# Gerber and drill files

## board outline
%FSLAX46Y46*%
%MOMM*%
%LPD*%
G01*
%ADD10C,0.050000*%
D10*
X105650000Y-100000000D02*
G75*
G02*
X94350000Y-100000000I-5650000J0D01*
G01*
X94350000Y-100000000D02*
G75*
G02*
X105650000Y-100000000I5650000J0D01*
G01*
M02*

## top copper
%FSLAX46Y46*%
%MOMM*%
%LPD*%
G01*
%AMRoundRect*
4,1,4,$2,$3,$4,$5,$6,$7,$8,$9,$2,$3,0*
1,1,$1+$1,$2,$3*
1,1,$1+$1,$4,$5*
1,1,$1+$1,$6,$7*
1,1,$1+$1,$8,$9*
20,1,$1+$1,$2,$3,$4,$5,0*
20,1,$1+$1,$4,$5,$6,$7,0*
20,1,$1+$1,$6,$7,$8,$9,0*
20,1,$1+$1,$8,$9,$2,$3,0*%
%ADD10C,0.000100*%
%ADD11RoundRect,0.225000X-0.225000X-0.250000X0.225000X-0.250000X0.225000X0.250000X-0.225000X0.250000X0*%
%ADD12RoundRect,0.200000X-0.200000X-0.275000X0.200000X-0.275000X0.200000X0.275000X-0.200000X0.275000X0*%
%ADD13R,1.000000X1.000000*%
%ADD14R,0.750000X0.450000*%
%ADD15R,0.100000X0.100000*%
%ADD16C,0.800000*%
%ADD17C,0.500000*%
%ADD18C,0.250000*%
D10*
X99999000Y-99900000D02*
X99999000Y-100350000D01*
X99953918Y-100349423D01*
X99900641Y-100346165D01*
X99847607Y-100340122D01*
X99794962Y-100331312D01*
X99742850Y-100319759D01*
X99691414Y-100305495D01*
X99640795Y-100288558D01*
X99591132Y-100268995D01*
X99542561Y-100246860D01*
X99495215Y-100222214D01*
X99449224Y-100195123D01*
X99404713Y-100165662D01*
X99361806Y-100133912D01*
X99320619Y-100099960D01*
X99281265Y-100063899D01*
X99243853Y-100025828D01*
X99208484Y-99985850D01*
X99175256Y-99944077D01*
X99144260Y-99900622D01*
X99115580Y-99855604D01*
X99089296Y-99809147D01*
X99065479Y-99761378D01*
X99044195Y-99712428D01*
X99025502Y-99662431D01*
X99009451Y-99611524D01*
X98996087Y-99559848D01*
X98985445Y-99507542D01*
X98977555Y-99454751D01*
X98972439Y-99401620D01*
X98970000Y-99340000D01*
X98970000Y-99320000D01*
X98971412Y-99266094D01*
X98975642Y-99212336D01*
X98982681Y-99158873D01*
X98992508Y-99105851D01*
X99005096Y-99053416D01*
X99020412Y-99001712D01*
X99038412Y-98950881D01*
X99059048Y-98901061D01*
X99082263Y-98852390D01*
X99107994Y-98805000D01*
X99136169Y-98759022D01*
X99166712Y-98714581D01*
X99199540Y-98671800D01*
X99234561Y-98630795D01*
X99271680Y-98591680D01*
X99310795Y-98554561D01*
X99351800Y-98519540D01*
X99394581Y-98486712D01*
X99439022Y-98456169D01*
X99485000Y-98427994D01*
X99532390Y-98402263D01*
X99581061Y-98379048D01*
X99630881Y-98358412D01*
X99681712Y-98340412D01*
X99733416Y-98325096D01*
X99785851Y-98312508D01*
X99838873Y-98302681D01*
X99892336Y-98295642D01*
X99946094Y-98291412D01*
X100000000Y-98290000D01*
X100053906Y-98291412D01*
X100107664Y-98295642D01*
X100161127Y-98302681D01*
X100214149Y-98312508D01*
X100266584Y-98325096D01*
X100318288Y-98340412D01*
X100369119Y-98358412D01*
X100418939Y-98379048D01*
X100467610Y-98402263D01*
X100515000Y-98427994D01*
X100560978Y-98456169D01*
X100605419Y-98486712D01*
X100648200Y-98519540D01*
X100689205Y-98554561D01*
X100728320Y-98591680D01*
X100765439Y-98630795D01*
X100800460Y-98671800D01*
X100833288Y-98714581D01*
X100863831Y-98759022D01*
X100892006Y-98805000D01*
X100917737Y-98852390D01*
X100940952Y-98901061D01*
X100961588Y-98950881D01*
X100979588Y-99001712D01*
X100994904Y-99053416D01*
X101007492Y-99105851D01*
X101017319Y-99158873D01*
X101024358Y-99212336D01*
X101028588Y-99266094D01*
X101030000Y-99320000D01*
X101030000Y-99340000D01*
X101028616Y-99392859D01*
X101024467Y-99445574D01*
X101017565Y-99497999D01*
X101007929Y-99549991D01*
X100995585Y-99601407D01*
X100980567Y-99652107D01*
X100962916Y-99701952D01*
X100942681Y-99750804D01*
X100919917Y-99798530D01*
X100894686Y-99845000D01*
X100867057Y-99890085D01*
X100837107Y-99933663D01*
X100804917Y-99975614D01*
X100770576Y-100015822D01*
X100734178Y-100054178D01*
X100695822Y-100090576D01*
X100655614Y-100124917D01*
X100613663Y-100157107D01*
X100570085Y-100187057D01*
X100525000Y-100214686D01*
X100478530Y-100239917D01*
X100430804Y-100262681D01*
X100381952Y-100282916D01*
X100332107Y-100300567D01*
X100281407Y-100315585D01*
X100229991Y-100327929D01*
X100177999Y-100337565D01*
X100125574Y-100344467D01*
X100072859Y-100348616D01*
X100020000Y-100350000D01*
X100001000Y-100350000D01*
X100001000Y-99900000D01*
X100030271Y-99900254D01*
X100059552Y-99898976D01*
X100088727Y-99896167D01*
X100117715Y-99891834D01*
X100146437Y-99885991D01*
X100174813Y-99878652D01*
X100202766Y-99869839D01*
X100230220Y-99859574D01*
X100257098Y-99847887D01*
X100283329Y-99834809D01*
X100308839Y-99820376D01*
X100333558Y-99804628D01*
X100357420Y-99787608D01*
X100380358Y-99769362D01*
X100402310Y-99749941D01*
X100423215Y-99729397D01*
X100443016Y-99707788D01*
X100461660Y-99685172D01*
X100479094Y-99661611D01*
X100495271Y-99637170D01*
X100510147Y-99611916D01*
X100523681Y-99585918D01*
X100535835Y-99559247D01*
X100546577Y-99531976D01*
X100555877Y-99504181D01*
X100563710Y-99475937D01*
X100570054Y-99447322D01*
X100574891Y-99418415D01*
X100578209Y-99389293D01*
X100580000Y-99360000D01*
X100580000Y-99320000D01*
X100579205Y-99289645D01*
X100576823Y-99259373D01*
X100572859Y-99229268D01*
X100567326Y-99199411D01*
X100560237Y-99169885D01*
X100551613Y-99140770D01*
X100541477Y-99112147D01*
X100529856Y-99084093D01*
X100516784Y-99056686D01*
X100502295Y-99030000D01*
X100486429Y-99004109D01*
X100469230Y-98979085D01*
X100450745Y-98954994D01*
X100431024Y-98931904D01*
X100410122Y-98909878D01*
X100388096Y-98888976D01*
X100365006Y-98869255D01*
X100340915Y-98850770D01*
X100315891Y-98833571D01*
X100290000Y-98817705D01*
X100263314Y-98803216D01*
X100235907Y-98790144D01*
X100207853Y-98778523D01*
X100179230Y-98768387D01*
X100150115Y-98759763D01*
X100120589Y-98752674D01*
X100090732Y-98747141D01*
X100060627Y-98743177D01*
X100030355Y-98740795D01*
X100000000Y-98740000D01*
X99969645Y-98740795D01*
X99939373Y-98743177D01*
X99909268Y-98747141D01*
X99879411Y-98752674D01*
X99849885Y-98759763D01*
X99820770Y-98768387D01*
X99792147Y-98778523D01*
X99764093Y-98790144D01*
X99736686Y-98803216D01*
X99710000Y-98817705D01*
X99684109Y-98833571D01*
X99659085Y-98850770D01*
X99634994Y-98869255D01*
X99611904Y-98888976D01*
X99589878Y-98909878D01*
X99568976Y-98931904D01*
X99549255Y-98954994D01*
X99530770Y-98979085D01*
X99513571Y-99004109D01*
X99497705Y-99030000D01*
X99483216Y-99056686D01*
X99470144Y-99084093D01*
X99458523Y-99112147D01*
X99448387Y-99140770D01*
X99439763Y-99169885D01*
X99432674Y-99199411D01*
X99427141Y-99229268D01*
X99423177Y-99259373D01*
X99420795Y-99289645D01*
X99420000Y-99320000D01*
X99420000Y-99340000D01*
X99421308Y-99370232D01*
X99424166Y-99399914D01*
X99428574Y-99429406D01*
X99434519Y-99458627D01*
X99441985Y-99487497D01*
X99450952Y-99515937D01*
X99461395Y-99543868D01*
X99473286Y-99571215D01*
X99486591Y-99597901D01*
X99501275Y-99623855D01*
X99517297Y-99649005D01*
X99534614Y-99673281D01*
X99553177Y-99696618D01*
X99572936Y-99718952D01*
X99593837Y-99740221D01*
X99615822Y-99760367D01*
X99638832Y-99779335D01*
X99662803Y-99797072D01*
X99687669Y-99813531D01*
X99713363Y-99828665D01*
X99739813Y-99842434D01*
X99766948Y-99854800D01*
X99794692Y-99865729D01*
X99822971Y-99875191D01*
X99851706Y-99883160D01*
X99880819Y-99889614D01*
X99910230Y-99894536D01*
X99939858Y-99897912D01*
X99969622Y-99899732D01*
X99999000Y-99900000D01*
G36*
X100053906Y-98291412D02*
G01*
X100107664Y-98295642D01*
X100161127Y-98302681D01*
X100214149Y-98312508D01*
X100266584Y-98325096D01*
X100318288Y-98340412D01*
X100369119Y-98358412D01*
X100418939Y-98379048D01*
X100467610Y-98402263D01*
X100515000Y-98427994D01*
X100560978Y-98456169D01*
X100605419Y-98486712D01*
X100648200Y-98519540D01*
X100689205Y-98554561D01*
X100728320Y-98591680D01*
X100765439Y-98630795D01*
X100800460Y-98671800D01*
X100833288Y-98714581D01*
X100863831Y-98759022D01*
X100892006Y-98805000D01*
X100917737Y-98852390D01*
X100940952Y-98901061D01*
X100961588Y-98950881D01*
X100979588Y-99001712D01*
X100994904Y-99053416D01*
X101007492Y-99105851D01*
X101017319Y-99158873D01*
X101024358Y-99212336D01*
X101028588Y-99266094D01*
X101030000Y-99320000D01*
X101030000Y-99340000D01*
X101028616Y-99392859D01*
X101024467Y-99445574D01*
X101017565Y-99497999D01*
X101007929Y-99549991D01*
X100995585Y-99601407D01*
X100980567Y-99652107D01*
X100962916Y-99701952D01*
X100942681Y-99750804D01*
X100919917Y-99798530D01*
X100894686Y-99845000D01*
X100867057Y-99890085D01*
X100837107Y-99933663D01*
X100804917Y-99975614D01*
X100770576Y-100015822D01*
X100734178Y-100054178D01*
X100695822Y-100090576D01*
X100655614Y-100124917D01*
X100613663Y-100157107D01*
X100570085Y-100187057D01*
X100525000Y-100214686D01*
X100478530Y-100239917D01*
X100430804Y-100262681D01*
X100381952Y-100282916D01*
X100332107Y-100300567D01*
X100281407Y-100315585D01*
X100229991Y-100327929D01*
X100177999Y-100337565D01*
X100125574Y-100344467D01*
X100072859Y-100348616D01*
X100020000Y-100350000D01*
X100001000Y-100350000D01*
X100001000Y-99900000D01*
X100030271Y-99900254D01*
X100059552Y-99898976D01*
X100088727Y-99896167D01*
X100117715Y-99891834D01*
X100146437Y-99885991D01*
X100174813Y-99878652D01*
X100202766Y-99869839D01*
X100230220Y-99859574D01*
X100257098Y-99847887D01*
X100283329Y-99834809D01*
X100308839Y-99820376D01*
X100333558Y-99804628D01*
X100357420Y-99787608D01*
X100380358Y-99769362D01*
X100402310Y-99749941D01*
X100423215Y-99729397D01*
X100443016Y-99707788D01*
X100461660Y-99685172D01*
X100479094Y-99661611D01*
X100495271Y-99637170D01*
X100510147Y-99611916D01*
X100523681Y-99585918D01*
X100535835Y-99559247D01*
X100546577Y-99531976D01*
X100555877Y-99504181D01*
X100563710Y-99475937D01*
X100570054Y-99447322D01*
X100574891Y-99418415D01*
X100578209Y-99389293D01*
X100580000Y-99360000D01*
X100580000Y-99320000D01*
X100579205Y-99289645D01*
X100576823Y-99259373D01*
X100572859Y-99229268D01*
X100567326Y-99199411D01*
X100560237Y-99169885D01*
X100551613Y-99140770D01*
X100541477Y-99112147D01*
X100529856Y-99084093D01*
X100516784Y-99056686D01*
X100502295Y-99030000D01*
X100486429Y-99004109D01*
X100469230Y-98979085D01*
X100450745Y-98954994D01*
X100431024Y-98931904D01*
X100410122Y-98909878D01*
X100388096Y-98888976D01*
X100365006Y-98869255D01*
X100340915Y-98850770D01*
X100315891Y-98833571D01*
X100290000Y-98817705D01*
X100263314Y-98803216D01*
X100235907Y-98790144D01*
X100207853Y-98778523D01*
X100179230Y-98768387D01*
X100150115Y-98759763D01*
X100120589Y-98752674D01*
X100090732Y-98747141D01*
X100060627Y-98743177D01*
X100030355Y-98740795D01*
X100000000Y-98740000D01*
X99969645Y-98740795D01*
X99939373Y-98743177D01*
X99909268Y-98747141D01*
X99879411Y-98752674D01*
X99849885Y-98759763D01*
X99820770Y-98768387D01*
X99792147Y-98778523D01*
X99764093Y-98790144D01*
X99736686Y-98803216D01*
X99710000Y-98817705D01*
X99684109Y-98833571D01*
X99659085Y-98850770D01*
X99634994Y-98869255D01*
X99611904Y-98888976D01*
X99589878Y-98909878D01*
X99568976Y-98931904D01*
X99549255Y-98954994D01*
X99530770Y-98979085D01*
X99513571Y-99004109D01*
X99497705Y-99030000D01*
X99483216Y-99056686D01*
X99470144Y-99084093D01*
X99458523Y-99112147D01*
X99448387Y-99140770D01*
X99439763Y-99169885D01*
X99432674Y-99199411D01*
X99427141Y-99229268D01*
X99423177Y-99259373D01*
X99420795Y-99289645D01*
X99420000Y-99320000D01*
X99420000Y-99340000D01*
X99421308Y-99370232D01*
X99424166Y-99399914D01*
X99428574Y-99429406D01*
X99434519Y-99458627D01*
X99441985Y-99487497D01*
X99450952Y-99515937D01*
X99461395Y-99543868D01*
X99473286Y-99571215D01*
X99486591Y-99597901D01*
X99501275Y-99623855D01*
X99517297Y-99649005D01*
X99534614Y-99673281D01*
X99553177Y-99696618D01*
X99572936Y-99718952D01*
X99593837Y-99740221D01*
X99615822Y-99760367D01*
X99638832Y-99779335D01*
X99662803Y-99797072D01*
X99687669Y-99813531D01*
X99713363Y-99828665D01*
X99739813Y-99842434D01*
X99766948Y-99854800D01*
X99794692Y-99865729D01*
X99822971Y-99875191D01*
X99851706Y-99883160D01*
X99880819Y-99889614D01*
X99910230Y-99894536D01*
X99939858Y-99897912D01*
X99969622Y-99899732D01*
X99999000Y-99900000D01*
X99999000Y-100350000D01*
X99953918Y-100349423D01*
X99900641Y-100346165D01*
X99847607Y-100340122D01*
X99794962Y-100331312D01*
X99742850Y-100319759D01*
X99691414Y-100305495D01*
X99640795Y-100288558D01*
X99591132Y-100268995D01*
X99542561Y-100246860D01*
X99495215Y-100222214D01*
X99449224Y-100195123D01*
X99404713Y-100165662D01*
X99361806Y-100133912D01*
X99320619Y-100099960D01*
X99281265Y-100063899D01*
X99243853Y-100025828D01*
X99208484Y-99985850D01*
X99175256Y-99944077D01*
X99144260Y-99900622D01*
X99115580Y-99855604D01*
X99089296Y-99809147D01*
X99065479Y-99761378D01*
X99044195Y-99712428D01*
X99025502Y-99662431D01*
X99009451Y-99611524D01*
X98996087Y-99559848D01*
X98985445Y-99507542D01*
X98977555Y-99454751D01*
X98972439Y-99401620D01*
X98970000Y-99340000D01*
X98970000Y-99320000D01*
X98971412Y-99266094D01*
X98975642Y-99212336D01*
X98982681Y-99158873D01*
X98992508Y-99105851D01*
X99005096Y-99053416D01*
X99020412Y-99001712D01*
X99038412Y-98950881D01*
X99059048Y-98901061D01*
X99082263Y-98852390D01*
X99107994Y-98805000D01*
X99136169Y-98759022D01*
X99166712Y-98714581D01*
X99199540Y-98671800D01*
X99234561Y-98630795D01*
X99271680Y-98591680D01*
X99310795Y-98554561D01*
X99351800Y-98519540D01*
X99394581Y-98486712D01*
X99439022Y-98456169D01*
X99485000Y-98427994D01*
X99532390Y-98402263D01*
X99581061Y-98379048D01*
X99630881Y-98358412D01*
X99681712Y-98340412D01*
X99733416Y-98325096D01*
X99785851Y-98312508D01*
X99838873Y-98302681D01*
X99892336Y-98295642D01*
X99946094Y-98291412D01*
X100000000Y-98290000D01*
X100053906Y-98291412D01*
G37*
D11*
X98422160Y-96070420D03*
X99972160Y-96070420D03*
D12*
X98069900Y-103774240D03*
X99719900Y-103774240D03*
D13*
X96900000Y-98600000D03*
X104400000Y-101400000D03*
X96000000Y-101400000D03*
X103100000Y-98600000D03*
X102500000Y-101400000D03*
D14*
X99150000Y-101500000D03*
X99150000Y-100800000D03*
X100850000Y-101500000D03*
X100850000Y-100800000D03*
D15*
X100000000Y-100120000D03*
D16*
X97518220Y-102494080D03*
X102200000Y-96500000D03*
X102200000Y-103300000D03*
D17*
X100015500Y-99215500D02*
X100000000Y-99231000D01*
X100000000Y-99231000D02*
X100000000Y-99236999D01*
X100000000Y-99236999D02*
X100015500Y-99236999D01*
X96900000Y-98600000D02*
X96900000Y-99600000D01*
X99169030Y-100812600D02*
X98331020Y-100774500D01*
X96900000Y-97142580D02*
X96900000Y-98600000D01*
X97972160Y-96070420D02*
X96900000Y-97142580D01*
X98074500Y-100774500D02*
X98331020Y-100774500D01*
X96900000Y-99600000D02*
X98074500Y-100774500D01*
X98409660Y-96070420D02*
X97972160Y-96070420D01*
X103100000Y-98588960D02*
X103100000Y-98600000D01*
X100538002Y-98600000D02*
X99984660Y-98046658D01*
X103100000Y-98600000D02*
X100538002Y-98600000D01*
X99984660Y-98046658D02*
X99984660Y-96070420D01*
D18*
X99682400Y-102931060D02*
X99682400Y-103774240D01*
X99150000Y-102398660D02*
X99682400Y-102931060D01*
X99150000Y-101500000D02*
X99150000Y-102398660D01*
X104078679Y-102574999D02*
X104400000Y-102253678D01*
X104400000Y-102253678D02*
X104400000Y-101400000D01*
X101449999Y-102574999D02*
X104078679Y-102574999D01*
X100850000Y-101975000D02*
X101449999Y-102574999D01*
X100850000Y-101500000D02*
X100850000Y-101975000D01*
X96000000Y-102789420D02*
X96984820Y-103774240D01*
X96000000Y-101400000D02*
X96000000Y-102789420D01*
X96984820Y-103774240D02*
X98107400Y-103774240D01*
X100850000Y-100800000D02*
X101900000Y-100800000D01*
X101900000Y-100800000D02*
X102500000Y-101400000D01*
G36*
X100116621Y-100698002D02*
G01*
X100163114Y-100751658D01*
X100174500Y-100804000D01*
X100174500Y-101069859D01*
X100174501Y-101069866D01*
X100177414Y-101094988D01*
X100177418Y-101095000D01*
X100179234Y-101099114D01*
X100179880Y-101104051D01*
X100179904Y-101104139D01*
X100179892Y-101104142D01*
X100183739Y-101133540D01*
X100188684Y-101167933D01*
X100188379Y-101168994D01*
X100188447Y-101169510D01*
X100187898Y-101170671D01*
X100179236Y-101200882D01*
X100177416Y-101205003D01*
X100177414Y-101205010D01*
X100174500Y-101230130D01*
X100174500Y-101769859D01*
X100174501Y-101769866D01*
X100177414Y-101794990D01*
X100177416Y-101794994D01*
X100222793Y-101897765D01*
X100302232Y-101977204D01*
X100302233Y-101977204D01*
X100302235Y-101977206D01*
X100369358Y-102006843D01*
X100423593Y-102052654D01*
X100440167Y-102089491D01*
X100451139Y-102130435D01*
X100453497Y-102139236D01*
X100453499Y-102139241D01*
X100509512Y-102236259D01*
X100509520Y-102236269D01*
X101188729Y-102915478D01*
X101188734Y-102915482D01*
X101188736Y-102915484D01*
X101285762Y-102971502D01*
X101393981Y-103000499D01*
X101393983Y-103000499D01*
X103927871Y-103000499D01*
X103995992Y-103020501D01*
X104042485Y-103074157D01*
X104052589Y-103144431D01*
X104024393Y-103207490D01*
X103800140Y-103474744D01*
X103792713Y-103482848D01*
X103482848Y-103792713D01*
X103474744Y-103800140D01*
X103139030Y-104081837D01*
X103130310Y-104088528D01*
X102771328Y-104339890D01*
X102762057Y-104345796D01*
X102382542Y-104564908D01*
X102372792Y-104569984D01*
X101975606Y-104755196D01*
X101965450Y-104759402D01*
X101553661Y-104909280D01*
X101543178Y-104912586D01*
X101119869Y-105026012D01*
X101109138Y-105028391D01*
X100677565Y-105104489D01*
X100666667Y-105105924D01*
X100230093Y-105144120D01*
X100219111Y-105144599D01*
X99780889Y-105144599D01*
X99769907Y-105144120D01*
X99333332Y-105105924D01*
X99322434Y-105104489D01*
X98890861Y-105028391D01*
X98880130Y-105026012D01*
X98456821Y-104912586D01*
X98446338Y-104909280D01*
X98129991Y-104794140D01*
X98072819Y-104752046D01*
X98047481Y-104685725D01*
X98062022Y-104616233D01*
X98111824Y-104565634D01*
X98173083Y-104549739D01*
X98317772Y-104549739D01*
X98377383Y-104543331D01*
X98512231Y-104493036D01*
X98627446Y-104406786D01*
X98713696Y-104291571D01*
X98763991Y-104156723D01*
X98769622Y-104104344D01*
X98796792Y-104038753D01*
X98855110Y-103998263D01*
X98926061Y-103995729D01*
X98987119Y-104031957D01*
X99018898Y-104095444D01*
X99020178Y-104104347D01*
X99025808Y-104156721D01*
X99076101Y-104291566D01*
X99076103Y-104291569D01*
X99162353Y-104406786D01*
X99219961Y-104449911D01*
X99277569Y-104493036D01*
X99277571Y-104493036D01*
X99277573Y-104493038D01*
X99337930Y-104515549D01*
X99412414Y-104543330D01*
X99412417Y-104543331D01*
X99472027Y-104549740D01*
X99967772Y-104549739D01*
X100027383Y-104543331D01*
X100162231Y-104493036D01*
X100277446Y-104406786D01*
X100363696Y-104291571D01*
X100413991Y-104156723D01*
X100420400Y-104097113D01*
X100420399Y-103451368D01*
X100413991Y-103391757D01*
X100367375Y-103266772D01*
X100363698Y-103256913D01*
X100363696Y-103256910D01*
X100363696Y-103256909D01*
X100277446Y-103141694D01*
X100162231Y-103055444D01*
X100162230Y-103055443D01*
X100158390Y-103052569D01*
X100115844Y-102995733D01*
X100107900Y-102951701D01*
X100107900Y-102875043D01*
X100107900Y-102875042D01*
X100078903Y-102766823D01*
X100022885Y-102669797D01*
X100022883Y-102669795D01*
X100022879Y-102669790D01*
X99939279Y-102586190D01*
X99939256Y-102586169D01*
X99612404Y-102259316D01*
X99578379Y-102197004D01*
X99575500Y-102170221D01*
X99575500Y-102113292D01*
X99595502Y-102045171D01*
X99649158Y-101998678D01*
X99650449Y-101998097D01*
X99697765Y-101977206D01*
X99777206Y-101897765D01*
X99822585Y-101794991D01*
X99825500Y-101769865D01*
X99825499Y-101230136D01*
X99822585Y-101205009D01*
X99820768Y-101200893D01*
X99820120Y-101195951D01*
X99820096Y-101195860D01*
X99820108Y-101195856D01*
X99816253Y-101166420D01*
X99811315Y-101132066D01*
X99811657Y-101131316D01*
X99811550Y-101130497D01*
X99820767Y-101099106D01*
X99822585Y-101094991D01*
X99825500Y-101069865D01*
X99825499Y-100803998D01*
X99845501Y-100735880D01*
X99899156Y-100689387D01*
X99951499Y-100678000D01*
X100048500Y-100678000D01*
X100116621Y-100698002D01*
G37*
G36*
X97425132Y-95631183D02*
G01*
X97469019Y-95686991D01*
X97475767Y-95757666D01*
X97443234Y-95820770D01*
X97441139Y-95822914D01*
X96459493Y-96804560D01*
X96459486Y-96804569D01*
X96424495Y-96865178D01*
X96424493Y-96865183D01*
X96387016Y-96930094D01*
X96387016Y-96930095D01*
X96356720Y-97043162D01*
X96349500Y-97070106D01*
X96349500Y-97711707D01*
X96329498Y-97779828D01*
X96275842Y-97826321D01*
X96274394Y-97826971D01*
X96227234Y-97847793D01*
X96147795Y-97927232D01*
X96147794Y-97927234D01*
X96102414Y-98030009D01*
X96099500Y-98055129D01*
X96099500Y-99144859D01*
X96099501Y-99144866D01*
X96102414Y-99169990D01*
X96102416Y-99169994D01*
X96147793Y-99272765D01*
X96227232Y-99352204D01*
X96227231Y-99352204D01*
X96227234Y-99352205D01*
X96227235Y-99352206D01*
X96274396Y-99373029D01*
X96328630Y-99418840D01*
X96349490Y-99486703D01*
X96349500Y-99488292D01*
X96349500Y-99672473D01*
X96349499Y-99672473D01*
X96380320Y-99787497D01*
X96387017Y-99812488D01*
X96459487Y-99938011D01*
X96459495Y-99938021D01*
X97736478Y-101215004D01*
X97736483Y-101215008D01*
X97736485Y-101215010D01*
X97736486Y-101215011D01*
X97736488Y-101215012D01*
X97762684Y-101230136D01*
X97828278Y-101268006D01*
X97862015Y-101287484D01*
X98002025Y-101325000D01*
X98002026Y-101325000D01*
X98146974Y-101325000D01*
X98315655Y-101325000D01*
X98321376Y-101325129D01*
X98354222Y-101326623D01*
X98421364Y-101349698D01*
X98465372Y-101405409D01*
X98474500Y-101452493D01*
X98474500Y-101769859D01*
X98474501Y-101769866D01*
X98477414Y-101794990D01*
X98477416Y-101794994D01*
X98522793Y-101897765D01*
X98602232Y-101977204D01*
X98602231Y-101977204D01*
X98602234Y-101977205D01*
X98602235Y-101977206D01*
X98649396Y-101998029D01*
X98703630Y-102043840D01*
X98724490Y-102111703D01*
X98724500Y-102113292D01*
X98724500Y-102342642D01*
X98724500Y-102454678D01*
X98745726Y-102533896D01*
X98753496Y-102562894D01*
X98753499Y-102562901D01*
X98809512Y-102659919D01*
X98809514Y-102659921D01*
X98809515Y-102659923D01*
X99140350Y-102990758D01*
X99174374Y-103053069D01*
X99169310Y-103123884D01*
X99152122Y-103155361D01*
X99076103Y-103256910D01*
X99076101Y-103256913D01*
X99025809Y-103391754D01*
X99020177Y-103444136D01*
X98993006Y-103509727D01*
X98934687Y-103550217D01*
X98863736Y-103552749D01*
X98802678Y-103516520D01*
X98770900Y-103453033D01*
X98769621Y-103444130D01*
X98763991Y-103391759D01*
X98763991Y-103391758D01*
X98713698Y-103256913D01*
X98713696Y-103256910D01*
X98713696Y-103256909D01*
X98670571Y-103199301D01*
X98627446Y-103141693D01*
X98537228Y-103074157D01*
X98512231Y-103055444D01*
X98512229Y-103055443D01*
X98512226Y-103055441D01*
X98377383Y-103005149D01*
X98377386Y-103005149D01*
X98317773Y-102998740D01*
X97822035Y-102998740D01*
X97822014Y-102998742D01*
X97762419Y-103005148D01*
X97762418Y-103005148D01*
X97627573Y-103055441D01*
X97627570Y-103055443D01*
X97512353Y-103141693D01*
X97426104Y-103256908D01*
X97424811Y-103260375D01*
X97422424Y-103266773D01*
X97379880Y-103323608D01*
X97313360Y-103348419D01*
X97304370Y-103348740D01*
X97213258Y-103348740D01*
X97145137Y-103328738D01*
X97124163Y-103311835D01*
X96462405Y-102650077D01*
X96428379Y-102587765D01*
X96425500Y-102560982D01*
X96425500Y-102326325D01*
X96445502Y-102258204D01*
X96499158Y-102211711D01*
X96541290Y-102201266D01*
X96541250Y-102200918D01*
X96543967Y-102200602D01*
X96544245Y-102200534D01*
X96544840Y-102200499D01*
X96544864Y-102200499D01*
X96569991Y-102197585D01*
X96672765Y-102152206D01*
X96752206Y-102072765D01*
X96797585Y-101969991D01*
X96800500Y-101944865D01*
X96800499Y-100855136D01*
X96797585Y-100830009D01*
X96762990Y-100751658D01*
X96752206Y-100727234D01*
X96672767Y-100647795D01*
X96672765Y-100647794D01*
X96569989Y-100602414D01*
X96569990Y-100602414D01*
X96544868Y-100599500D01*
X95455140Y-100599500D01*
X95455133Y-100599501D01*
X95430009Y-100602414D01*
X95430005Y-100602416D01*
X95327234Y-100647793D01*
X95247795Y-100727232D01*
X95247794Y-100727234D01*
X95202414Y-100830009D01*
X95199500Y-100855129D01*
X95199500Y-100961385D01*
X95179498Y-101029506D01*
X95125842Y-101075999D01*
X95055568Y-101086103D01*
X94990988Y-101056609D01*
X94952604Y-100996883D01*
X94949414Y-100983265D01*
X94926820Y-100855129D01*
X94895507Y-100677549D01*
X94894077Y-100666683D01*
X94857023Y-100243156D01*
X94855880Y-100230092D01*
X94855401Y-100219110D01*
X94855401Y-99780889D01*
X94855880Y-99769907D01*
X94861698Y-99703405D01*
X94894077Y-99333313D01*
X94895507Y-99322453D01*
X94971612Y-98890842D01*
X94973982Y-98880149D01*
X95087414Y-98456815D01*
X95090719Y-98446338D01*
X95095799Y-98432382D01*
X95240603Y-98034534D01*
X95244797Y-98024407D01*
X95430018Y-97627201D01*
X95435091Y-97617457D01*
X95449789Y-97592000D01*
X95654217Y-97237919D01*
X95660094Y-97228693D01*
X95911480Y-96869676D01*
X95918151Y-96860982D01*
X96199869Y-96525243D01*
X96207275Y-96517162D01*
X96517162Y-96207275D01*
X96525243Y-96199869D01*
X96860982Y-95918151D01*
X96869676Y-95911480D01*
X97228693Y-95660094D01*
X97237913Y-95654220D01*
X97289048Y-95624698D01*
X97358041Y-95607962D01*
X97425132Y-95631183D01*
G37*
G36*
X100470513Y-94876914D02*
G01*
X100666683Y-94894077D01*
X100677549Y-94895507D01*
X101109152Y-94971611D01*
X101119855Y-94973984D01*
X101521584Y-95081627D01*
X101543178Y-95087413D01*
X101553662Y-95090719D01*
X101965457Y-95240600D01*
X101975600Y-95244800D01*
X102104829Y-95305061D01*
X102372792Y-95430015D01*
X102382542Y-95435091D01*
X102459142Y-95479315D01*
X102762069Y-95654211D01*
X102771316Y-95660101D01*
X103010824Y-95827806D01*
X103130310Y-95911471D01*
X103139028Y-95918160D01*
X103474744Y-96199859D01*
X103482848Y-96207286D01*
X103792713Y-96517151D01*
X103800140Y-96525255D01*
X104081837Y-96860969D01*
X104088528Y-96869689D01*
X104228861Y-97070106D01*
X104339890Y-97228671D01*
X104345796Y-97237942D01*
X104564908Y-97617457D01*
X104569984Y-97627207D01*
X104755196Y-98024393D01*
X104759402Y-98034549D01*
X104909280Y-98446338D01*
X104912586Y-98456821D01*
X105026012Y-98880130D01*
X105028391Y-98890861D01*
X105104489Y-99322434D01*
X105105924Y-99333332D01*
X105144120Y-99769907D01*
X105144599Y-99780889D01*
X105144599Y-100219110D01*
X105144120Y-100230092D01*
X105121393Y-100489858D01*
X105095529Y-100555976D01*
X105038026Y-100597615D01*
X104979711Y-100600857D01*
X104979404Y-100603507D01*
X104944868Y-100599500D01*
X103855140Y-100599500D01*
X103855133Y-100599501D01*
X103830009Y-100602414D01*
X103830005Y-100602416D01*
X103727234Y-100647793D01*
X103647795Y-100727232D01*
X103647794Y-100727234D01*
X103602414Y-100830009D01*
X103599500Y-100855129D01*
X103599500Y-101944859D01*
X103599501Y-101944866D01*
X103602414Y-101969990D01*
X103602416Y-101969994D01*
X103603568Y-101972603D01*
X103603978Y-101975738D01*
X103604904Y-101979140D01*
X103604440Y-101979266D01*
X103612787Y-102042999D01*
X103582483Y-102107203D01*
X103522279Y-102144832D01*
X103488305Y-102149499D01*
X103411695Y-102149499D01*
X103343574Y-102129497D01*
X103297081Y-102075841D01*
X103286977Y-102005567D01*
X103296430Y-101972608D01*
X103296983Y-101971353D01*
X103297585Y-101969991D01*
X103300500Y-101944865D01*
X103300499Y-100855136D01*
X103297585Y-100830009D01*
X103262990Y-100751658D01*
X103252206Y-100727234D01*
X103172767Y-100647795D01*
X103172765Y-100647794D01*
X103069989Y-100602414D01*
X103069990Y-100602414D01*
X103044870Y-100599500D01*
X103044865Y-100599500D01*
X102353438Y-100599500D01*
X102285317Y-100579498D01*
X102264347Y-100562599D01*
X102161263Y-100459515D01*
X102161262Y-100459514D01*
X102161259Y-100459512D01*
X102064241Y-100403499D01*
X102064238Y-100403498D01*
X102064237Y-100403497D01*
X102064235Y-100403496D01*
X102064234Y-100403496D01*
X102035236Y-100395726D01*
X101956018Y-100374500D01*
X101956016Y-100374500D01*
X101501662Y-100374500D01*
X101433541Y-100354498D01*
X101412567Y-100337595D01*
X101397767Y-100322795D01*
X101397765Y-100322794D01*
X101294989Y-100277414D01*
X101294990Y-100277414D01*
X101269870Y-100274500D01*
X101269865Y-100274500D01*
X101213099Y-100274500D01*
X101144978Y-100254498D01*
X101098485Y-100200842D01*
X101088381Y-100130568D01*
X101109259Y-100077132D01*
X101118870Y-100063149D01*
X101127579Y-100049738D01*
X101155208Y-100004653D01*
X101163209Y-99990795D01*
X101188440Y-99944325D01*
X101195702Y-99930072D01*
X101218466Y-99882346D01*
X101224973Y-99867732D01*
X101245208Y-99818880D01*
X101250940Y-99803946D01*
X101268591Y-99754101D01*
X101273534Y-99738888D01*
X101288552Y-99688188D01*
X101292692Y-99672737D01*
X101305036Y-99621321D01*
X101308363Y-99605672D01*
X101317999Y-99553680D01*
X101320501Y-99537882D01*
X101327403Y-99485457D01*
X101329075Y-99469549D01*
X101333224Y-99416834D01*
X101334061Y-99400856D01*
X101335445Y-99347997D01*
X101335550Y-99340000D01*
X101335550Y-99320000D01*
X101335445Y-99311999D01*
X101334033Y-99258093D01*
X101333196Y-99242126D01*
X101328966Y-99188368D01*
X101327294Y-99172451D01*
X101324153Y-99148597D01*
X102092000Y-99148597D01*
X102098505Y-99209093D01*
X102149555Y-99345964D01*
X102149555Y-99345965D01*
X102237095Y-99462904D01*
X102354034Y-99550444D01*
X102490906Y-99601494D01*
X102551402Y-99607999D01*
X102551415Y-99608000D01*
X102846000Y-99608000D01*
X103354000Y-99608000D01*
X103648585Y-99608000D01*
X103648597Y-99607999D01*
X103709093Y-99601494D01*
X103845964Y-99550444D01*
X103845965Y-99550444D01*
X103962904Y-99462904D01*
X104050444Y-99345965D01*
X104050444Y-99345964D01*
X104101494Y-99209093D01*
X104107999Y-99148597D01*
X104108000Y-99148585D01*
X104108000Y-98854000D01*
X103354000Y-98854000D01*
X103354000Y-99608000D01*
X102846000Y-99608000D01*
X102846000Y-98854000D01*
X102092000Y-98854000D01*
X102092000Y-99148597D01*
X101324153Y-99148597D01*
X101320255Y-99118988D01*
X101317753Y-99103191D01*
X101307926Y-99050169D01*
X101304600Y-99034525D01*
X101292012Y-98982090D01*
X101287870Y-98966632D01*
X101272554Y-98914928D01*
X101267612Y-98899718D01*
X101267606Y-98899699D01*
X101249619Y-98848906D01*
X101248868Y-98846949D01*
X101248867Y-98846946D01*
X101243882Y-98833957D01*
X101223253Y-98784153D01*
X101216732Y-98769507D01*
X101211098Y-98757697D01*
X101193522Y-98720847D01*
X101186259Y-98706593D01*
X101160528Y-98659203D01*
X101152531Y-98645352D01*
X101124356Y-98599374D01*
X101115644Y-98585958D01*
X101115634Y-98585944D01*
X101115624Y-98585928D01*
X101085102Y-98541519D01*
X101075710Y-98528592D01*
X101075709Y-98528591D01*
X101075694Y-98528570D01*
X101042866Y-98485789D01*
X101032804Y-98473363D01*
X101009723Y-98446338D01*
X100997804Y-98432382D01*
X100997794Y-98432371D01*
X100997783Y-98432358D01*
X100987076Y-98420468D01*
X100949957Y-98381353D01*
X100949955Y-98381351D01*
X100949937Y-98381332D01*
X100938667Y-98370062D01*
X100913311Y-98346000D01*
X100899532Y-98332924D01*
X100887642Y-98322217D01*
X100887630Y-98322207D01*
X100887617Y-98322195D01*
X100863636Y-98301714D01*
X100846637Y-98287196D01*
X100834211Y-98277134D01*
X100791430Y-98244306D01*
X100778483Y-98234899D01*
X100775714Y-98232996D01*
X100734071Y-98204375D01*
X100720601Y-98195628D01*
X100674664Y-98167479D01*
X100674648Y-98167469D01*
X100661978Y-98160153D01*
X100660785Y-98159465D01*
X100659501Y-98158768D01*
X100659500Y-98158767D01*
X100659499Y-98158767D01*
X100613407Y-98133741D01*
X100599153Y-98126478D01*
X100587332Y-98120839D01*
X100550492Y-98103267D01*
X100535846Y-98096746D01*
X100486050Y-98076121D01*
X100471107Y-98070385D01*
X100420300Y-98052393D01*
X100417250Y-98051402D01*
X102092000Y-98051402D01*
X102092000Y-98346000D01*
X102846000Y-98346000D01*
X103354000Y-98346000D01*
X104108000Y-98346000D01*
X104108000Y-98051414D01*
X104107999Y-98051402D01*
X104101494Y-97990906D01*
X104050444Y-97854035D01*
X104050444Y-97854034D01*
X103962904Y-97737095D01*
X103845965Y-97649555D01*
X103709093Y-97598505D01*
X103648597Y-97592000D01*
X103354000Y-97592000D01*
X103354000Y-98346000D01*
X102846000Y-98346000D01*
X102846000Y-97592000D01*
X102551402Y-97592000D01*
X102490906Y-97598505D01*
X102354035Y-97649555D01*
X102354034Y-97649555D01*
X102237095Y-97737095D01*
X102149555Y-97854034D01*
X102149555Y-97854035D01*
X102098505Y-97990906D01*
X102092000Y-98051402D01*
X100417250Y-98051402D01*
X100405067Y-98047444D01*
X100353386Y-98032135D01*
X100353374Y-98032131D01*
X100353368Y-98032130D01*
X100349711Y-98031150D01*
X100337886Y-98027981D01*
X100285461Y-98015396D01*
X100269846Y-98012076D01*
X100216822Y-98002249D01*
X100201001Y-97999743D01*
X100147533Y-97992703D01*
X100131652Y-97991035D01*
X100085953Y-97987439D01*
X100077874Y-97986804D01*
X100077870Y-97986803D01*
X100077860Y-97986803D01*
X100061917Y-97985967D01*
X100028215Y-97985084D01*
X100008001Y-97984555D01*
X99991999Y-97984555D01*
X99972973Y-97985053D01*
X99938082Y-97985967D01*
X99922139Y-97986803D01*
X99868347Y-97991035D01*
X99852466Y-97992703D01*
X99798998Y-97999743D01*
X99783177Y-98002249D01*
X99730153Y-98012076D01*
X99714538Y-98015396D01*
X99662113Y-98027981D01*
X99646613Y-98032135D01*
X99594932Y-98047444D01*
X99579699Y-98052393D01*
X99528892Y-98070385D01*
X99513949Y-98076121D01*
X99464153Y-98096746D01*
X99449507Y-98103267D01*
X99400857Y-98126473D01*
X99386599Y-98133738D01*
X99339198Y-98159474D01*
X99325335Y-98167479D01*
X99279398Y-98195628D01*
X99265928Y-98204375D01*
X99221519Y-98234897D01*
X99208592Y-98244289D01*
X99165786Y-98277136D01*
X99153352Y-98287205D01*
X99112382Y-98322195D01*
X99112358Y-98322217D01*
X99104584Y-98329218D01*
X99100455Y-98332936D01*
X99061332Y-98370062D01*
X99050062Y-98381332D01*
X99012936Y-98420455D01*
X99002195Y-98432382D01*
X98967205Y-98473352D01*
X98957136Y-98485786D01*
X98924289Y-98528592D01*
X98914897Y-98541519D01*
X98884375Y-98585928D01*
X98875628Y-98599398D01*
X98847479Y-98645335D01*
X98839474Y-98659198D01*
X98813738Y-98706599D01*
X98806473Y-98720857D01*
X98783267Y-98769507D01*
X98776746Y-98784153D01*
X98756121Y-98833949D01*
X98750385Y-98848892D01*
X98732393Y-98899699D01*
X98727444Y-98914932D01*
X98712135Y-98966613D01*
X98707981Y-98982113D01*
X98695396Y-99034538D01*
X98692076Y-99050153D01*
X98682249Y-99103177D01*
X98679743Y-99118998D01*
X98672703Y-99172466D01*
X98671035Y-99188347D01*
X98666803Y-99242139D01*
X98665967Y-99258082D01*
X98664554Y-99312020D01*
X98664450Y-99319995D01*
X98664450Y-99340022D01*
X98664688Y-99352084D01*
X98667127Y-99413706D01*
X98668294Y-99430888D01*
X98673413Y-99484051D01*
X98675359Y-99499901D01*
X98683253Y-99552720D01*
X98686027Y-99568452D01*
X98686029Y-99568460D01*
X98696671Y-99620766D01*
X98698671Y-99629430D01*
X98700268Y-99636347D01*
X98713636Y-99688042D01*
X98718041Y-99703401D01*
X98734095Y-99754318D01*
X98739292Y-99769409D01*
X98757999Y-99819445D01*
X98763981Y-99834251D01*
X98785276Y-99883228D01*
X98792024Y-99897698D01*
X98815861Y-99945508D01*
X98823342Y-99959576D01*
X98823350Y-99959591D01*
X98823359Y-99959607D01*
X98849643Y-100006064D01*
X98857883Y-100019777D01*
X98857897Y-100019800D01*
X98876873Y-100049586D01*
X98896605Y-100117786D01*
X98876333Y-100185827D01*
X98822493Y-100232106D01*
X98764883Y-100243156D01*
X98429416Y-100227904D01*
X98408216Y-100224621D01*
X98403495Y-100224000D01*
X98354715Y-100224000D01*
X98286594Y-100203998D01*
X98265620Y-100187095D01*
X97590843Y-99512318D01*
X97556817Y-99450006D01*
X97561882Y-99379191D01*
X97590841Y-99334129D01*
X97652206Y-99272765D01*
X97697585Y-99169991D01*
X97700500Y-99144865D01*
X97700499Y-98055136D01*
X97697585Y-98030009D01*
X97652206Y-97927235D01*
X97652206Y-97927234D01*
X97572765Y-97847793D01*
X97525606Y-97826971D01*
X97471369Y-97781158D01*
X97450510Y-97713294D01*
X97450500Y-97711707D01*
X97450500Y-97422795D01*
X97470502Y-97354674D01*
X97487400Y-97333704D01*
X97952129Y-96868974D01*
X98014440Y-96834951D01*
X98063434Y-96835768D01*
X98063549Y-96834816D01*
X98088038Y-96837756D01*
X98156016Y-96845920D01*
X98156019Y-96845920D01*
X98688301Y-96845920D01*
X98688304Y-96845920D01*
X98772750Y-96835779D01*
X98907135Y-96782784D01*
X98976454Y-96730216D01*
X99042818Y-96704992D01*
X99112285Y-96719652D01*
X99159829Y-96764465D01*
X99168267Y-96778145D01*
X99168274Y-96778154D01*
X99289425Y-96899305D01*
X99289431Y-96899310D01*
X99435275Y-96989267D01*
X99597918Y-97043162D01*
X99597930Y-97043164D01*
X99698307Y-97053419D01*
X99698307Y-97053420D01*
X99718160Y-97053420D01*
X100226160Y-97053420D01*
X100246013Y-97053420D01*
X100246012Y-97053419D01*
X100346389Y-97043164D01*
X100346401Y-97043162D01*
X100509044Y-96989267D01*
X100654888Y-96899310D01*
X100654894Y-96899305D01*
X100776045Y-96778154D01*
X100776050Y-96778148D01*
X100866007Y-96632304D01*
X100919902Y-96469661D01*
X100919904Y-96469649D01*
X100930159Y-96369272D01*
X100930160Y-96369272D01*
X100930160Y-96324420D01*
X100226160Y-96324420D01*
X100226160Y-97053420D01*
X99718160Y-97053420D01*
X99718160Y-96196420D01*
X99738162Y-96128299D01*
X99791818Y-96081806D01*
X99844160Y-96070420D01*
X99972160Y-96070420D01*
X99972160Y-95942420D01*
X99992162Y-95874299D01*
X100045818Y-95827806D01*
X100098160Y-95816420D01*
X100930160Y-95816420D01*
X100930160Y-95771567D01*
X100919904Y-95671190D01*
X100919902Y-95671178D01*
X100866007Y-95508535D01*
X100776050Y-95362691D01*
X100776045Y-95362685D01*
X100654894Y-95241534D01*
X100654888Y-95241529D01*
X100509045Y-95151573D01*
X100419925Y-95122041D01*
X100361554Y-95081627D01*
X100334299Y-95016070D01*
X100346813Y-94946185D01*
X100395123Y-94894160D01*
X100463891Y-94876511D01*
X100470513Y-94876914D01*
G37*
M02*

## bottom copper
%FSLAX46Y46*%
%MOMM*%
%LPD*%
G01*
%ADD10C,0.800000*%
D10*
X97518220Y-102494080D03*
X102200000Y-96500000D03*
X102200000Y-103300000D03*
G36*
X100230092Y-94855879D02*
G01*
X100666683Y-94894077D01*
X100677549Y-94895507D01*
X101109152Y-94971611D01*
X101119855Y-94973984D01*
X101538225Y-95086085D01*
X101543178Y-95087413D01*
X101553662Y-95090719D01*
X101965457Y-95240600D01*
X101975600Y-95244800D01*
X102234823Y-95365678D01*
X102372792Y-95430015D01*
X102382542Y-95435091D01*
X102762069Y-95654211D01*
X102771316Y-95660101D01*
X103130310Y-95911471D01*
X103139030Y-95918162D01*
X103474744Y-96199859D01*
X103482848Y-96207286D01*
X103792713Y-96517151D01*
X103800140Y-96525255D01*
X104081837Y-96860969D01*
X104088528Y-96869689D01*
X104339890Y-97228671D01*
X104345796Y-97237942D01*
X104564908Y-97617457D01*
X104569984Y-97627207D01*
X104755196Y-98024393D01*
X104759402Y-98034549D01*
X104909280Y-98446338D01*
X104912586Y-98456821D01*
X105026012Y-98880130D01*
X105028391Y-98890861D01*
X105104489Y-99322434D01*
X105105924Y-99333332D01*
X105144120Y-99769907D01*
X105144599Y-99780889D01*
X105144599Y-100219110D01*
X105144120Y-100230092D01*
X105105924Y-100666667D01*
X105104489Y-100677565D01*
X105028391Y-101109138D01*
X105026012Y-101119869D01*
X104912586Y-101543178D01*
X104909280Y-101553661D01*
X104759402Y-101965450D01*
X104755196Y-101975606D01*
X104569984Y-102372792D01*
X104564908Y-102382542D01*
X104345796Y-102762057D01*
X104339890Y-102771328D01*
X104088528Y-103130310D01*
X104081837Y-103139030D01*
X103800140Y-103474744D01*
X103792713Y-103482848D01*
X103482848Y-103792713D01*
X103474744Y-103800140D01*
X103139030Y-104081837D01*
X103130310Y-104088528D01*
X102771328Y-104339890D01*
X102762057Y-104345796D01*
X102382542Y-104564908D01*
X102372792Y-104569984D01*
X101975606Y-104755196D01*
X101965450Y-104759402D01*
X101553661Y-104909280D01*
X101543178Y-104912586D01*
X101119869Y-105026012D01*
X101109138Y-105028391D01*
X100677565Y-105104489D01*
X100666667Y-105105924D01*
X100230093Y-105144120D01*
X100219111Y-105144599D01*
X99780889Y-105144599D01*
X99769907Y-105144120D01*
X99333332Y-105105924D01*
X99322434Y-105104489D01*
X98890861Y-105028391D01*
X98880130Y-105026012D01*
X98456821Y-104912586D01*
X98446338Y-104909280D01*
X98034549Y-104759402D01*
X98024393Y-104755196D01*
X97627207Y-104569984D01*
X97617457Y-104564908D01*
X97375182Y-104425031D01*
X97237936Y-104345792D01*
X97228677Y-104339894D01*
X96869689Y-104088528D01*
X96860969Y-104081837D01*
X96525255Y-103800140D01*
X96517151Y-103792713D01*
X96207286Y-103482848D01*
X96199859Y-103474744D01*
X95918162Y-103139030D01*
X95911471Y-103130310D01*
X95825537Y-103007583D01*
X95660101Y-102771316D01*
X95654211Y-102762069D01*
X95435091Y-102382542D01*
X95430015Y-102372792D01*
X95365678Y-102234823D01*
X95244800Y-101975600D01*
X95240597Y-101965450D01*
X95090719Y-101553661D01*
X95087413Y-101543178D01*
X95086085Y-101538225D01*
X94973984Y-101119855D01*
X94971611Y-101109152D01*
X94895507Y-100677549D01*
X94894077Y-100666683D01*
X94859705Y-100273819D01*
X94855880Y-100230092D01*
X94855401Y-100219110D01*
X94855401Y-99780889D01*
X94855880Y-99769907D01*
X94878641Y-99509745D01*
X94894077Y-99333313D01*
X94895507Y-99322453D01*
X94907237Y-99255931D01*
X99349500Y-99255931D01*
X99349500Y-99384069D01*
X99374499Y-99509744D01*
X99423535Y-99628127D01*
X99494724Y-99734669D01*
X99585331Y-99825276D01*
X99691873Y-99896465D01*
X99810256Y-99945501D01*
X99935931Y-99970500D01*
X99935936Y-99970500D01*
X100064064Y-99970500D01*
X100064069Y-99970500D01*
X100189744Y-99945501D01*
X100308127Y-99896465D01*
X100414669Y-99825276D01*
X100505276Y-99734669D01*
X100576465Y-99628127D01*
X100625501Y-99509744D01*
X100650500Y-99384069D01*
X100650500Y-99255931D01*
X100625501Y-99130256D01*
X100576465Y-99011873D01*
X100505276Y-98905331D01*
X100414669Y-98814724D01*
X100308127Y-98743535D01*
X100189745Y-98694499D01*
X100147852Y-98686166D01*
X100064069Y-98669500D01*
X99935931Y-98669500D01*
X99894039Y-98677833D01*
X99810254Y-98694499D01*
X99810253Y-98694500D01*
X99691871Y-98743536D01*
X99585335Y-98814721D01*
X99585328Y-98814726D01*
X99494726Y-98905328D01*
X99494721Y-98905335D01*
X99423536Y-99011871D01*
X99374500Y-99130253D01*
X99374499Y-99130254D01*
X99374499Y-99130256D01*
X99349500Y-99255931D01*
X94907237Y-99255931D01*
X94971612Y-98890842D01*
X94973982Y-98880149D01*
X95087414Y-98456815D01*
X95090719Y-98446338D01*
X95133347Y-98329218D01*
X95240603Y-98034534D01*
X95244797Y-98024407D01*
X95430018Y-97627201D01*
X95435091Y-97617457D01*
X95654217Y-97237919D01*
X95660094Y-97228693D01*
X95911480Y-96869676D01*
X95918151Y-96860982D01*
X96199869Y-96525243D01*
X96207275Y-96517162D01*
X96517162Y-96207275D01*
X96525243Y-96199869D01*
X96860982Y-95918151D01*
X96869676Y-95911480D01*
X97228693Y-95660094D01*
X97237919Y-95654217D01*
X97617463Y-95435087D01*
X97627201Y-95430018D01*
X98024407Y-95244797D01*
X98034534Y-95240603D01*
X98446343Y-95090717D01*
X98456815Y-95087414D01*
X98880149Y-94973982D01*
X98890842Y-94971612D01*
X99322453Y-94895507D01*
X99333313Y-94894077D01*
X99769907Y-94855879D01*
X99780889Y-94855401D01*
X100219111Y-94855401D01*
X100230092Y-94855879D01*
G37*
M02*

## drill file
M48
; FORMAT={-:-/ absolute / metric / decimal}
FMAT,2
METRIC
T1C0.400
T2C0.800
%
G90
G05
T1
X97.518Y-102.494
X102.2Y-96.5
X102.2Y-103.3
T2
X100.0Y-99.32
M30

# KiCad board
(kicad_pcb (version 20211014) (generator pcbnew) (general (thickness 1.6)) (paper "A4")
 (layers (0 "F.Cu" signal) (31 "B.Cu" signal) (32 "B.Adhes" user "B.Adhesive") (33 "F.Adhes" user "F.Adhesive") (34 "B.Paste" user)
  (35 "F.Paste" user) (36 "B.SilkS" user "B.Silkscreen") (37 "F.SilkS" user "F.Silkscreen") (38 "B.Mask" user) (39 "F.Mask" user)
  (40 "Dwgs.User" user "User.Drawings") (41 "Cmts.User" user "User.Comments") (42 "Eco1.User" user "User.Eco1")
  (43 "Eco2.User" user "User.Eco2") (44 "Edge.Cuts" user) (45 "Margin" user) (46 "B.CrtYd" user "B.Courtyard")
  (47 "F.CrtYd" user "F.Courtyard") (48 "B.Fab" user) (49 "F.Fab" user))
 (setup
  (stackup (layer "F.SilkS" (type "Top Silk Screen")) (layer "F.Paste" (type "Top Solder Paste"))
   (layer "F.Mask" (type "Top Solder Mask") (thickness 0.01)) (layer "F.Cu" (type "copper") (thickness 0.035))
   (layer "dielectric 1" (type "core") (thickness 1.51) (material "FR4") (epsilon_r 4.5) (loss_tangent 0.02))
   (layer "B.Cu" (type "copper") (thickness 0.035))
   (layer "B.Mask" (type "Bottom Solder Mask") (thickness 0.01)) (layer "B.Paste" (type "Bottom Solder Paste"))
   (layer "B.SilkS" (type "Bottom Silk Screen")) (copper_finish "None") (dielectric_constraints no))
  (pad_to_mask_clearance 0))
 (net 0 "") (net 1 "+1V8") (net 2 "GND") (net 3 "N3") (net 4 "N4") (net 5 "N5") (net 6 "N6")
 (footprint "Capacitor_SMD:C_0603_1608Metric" (layer "F.Cu") (at 99.19716 96.07042)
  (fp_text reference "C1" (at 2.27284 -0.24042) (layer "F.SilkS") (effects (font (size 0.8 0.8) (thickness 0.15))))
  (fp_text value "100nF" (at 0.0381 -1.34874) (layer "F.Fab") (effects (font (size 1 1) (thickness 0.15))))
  (pad "1" smd roundrect (at -0.775 0) (size 0.9 0.95) (layers "F.Cu" "F.Paste" "F.Mask") (roundrect_rratio 0.25) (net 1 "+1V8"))
  (pad "2" smd roundrect (at 0.775 0) (size 0.9 0.95) (layers "F.Cu" "F.Paste" "F.Mask") (roundrect_rratio 0.25) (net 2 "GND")))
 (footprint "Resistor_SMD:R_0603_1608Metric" (layer "F.Cu") (at 98.8949 103.77424)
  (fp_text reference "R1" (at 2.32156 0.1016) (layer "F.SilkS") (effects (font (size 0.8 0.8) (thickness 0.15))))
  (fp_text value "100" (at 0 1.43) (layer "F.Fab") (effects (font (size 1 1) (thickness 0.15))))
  (pad "1" smd roundrect (at -0.825 0) (size 0.8 0.95) (layers "F.Cu" "F.Paste" "F.Mask") (roundrect_rratio 0.25) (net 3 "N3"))
  (pad "2" smd roundrect (at 0.825 0) (size 0.8 0.95) (layers "F.Cu" "F.Paste" "F.Mask") (roundrect_rratio 0.25) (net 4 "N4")))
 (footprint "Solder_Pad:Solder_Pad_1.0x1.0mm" (layer "F.Cu") (at 96.9 98.6)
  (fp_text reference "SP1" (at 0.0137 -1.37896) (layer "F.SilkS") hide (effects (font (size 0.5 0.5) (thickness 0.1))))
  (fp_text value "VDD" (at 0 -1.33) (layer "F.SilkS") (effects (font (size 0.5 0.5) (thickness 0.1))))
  (pad "1" smd rect locked (at 0 0) (size 1 1) (layers "F.Cu" "F.Mask") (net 1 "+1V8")))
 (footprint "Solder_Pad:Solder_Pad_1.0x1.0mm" (layer "F.Cu") (at 104.4 101.4)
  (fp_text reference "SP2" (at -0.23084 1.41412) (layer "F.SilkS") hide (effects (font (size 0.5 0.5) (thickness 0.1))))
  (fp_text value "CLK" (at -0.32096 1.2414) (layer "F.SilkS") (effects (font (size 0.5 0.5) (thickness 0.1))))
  (pad "1" smd rect locked (at 0 0) (size 1 1) (layers "F.Cu" "F.Mask") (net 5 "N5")))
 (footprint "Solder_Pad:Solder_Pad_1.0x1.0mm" (layer "F.Cu") (at 96 101.4)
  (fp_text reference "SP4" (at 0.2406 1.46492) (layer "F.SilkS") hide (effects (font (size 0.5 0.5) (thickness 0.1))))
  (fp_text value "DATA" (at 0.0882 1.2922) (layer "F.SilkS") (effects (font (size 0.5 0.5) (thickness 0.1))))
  (pad "1" smd rect locked (at 0 0) (size 1 1) (layers "F.Cu" "F.Mask") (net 3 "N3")))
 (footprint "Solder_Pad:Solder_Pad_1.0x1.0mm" (layer "F.Cu") (at 103.1 98.6)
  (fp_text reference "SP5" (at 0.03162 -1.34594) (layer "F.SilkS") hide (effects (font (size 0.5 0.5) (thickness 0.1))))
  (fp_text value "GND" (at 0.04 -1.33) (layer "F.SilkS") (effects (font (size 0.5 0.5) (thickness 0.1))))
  (pad "1" smd rect locked (at 0 0) (size 1 1) (layers "F.Cu" "F.Mask") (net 2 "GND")))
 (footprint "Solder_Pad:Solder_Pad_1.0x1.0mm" (layer "F.Cu") (at 102.5 101.4)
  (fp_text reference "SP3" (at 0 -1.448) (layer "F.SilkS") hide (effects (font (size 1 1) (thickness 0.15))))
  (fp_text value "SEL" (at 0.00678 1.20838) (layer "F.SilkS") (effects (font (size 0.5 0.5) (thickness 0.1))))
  (pad "1" smd rect locked (at 0 0) (size 1 1) (layers "F.Cu" "F.Mask") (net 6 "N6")))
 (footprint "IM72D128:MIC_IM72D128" (layer "F.Cu") (at 100 100 180)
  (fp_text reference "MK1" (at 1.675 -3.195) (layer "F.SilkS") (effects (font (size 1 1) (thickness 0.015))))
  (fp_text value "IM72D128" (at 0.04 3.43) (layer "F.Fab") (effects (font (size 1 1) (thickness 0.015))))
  (fp_poly
   (pts (xy 0.001 0.1) (xy 0.001 -0.35) (xy 0.046082 -0.349423) (xy 0.099359 -0.346165) (xy 0.152393 -0.340122) (xy 0.205038 -0.331312)
    (xy 0.25715 -0.319759) (xy 0.308586 -0.305495) (xy 0.359205 -0.288558) (xy 0.408868 -0.268995) (xy 0.457439 -0.24686)
    (xy 0.504785 -0.222214) (xy 0.550776 -0.195123) (xy 0.595287 -0.165662) (xy 0.638194 -0.133912) (xy 0.679381 -0.09996)
    (xy 0.718735 -0.063899) (xy 0.756147 -0.025828) (xy 0.791516 0.01415) (xy 0.824744 0.055923) (xy 0.85574 0.099378) (xy 0.88442 0.144396)
    (xy 0.910704 0.190853) (xy 0.934521 0.238622) (xy 0.955805 0.287572) (xy 0.974498 0.337569) (xy 0.990549 0.388476)
    (xy 1.003913 0.440152) (xy 1.014555 0.492458) (xy 1.022445 0.545249) (xy 1.027561 0.59838) (xy 1.03 0.66) (xy 1.03 0.68)
    (xy 1.028588 0.733906) (xy 1.024358 0.787664) (xy 1.017319 0.841127) (xy 1.007492 0.894149) (xy 0.994904 0.946584)
    (xy 0.979588 0.998288) (xy 0.961588 1.049119) (xy 0.940952 1.098939) (xy 0.917737 1.14761) (xy 0.892006 1.195) (xy 0.863831 1.240978)
    (xy 0.833288 1.285419) (xy 0.80046 1.3282) (xy 0.765439 1.369205) (xy 0.72832 1.40832) (xy 0.689205 1.445439) (xy 0.6482 1.48046)
    (xy 0.605419 1.513288) (xy 0.560978 1.543831) (xy 0.515 1.572006) (xy 0.46761 1.597737) (xy 0.418939 1.620952) (xy 0.369119 1.641588)
    (xy 0.318288 1.659588) (xy 0.266584 1.674904) (xy 0.214149 1.687492) (xy 0.161127 1.697319) (xy 0.107664 1.704358)
    (xy 0.053906 1.708588) (xy 0 1.71) (xy -0.053906 1.708588) (xy -0.107664 1.704358) (xy -0.161127 1.697319) (xy -0.214149 1.687492)
    (xy -0.266584 1.674904) (xy -0.318288 1.659588) (xy -0.369119 1.641588) (xy -0.418939 1.620952) (xy -0.46761 1.597737)
    (xy -0.515 1.572006) (xy -0.560978 1.543831) (xy -0.605419 1.513288) (xy -0.6482 1.48046) (xy -0.689205 1.445439) (xy -0.72832 1.40832)
    (xy -0.765439 1.369205) (xy -0.80046 1.3282) (xy -0.833288 1.285419) (xy -0.863831 1.240978) (xy -0.892006 1.195) (xy -0.917737 1.14761)
    (xy -0.940952 1.098939) (xy -0.961588 1.049119) (xy -0.979588 0.998288) (xy -0.994904 0.946584) (xy -1.007492 0.894149)
    (xy -1.017319 0.841127) (xy -1.024358 0.787664) (xy -1.028588 0.733906) (xy -1.03 0.68) (xy -1.03 0.66) (xy -1.028616 0.607141)
    (xy -1.024467 0.554426) (xy -1.017565 0.502001) (xy -1.007929 0.450009) (xy -0.995585 0.398593) (xy -0.980567 0.347893)
    (xy -0.962916 0.298048) (xy -0.942681 0.249196) (xy -0.919917 0.20147) (xy -0.894686 0.155) (xy -0.867057 0.109915)
    (xy -0.837107 0.066337) (xy -0.804917 0.024386) (xy -0.770576 -0.015822) (xy -0.734178 -0.054178) (xy -0.695822 -0.090576)
    (xy -0.655614 -0.124917) (xy -0.613663 -0.157107) (xy -0.570085 -0.187057) (xy -0.525 -0.214686) (xy -0.47853 -0.239917)
    (xy -0.430804 -0.262681) (xy -0.381952 -0.282916) (xy -0.332107 -0.300567) (xy -0.281407 -0.315585) (xy -0.229991 -0.327929)
    (xy -0.177999 -0.337565) (xy -0.125574 -0.344467) (xy -0.072859 -0.348616) (xy -0.02 -0.35) (xy -0.001 -0.35) (xy -0.001 0.1)
    (xy -0.030271 0.099746) (xy -0.059552 0.101024) (xy -0.088727 0.103833) (xy -0.117715 0.108166) (xy -0.146437 0.114009)
    (xy -0.174813 0.121348) (xy -0.202766 0.130161) (xy -0.23022 0.140426) (xy -0.257098 0.152113) (xy -0.283329 0.165191)
    (xy -0.308839 0.179624) (xy -0.333558 0.195372) (xy -0.35742 0.212392) (xy -0.380358 0.230638) (xy -0.40231 0.250059)
    (xy -0.423215 0.270603) (xy -0.443016 0.292212) (xy -0.46166 0.314828) (xy -0.479094 0.338389) (xy -0.495271 0.36283)
    (xy -0.510147 0.388084) (xy -0.523681 0.414082) (xy -0.535835 0.440753) (xy -0.546577 0.468024) (xy -0.555877 0.495819)
    (xy -0.56371 0.524063) (xy -0.570054 0.552678) (xy -0.574891 0.581585) (xy -0.578209 0.610707) (xy -0.58 0.64) (xy -0.58 0.68)
    (xy -0.579205 0.710355) (xy -0.576823 0.740627) (xy -0.572859 0.770732) (xy -0.567326 0.800589) (xy -0.560237 0.830115)
    (xy -0.551613 0.85923) (xy -0.541477 0.887853) (xy -0.529856 0.915907) (xy -0.516784 0.943314) (xy -0.502295 0.97)
    (xy -0.486429 0.995891) (xy -0.46923 1.020915) (xy -0.450745 1.045006) (xy -0.431024 1.068096) (xy -0.410122 1.090122)
    (xy -0.388096 1.111024) (xy -0.365006 1.130745) (xy -0.340915 1.14923) (xy -0.315891 1.166429) (xy -0.29 1.182295)
    (xy -0.263314 1.196784) (xy -0.235907 1.209856) (xy -0.207853 1.221477) (xy -0.17923 1.231613) (xy -0.150115 1.240237)
    (xy -0.120589 1.247326) (xy -0.090732 1.252859) (xy -0.060627 1.256823) (xy -0.030355 1.259205) (xy 0 1.26) (xy 0.030355 1.259205)
    (xy 0.060627 1.256823) (xy 0.090732 1.252859) (xy 0.120589 1.247326) (xy 0.150115 1.240237) (xy 0.17923 1.231613) (xy 0.207853 1.221477)
    (xy 0.235907 1.209856) (xy 0.263314 1.196784) (xy 0.29 1.182295) (xy 0.315891 1.166429) (xy 0.340915 1.14923) (xy 0.365006 1.130745)
    (xy 0.388096 1.111024) (xy 0.410122 1.090122) (xy 0.431024 1.068096) (xy 0.450745 1.045006) (xy 0.46923 1.020915) (xy 0.486429 0.995891)
    (xy 0.502295 0.97) (xy 0.516784 0.943314) (xy 0.529856 0.915907) (xy 0.541477 0.887853) (xy 0.551613 0.85923) (xy 0.560237 0.830115)
    (xy 0.567326 0.800589) (xy 0.572859 0.770732) (xy 0.576823 0.740627) (xy 0.579205 0.710355) (xy 0.58 0.68) (xy 0.58 0.66)
    (xy 0.578692 0.629768) (xy 0.575834 0.600086) (xy 0.571426 0.570594) (xy 0.565481 0.541373) (xy 0.558015 0.512503)
    (xy 0.549048 0.484063) (xy 0.538605 0.456132) (xy 0.526714 0.428785) (xy 0.513409 0.402099) (xy 0.498725 0.376145)
    (xy 0.482703 0.350995) (xy 0.465386 0.326719) (xy 0.446823 0.303382) (xy 0.427064 0.281048) (xy 0.406163 0.259779)
    (xy 0.384178 0.239633) (xy 0.361168 0.220665) (xy 0.337197 0.202928) (xy 0.312331 0.186469) (xy 0.286637 0.171335)
    (xy 0.260187 0.157566) (xy 0.233052 0.1452) (xy 0.205308 0.134271) (xy 0.177029 0.124809) (xy 0.148294 0.11684) (xy 0.119181 0.110386)
    (xy 0.08977 0.105464) (xy 0.060142 0.102088) (xy 0.030378 0.100268) (xy 0.001 0.1))
   (layer "F.Cu") (width 0.0001) (fill solid))
  (pad "" np_thru_hole circle (at 0 0.68 180) (size 0.8 0.8) (drill 0.8) (layers *.Cu *.Mask))
  (pad "1" smd rect (at 0.85 -1.5 180) (size 0.75 0.45) (layers "F.Cu" "F.Mask") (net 4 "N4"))
  (pad "2" smd rect (at 0.85 -0.8 180) (size 0.75 0.45) (layers "F.Cu" "F.Mask") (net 1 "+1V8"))
  (pad "3" smd rect (at -0.85 -1.5 180) (size 0.75 0.45) (layers "F.Cu" "F.Mask") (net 5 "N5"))
  (pad "4" smd rect (at -0.85 -0.8 180) (size 0.75 0.45) (layers "F.Cu" "F.Mask") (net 6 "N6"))
  (pad "5" smd rect (at 0 -0.12 180) (size 0.1 0.1) (layers "F.Cu") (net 2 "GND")))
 (gr_circle (center 100 100) (end 105.65 100) (layer "Edge.Cuts") (width 0.05) (fill none))
 (segment (start 100.0155 99.2155) (end 100 99.231) (width 0.5) (layer "F.Cu") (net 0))
 (segment (start 100 99.231) (end 100 99.236999) (width 0.5) (layer "F.Cu") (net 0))
 (segment (start 100 99.236999) (end 100.0155 99.236999) (width 0.5) (layer "F.Cu") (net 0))
 (segment (start 96.9 98.6) (end 96.9 99.6) (width 0.5) (layer "F.Cu") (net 1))
 (segment (start 99.16903 100.8126) (end 98.33102 100.7745) (width 0.5) (layer "F.Cu") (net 1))
 (segment (start 96.9 97.14258) (end 96.9 98.6) (width 0.5) (layer "F.Cu") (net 1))
 (segment (start 97.97216 96.07042) (end 96.9 97.14258) (width 0.5) (layer "F.Cu") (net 1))
 (segment (start 98.0745 100.7745) (end 98.33102 100.7745) (width 0.5) (layer "F.Cu") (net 1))
 (segment (start 96.9 99.6) (end 98.0745 100.7745) (width 0.5) (layer "F.Cu") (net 1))
 (segment (start 98.40966 96.07042) (end 97.97216 96.07042) (width 0.5) (layer "F.Cu") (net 1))
 (segment (start 103.1 98.58896) (end 103.1 98.6) (width 0.5) (layer "F.Cu") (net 2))
 (segment (start 100.538002 98.6) (end 99.98466 98.046658) (width 0.5) (layer "F.Cu") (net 2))
 (segment (start 103.1 98.6) (end 100.538002 98.6) (width 0.5) (layer "F.Cu") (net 2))
 (segment (start 99.98466 98.046658) (end 99.98466 96.07042) (width 0.5) (layer "F.Cu") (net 2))
 (via (at 97.51822 102.49408) (size 0.8) (drill 0.4) (layers "F.Cu" "B.Cu") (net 2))
 (via (at 102.2 96.5) (size 0.8) (drill 0.4) (layers "F.Cu" "B.Cu") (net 2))
 (via (at 102.2 103.3) (size 0.8) (drill 0.4) (layers "F.Cu" "B.Cu") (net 2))
 (segment (start 99.6824 102.93106) (end 99.6824 103.77424) (width 0.25) (layer "F.Cu") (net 4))
 (segment (start 99.15 102.39866) (end 99.6824 102.93106) (width 0.25) (layer "F.Cu") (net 4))
 (segment (start 99.15 101.5) (end 99.15 102.39866) (width 0.25) (layer "F.Cu") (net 4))
 (segment (start 104.078679 102.574999) (end 104.4 102.253678) (width 0.25) (layer "F.Cu") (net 5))
 (segment (start 104.4 102.253678) (end 104.4 101.4) (width 0.25) (layer "F.Cu") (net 5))
 (segment (start 101.449999 102.574999) (end 104.078679 102.574999) (width 0.25) (layer "F.Cu") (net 5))
 (segment (start 100.85 101.975) (end 101.449999 102.574999) (width 0.25) (layer "F.Cu") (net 5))
 (segment (start 100.85 101.5) (end 100.85 101.975) (width 0.25) (layer "F.Cu") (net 5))
 (segment (start 96 102.78942) (end 96.98482 103.77424) (width 0.25) (layer "F.Cu") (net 3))
 (segment (start 96 101.4) (end 96 102.78942) (width 0.25) (layer "F.Cu") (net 3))
 (segment (start 96.98482 103.77424) (end 98.1074 103.77424) (width 0.25) (layer "F.Cu") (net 3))
 (segment (start 100.85 100.8) (end 101.9 100.8) (width 0.25) (layer "F.Cu") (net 6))
 (segment (start 101.9 100.8) (end 102.5 101.4) (width 0.25) (layer "F.Cu") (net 6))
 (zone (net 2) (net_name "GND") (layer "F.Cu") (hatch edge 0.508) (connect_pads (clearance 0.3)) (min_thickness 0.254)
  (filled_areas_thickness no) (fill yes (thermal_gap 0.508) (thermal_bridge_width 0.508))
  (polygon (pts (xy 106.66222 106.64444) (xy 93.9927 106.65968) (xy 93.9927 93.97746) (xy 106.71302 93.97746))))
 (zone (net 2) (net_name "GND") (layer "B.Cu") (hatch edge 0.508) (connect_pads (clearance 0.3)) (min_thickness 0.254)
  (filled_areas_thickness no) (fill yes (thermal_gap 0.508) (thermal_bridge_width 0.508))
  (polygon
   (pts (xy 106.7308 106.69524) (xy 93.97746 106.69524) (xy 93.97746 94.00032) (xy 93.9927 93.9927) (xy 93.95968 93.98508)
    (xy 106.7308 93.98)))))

